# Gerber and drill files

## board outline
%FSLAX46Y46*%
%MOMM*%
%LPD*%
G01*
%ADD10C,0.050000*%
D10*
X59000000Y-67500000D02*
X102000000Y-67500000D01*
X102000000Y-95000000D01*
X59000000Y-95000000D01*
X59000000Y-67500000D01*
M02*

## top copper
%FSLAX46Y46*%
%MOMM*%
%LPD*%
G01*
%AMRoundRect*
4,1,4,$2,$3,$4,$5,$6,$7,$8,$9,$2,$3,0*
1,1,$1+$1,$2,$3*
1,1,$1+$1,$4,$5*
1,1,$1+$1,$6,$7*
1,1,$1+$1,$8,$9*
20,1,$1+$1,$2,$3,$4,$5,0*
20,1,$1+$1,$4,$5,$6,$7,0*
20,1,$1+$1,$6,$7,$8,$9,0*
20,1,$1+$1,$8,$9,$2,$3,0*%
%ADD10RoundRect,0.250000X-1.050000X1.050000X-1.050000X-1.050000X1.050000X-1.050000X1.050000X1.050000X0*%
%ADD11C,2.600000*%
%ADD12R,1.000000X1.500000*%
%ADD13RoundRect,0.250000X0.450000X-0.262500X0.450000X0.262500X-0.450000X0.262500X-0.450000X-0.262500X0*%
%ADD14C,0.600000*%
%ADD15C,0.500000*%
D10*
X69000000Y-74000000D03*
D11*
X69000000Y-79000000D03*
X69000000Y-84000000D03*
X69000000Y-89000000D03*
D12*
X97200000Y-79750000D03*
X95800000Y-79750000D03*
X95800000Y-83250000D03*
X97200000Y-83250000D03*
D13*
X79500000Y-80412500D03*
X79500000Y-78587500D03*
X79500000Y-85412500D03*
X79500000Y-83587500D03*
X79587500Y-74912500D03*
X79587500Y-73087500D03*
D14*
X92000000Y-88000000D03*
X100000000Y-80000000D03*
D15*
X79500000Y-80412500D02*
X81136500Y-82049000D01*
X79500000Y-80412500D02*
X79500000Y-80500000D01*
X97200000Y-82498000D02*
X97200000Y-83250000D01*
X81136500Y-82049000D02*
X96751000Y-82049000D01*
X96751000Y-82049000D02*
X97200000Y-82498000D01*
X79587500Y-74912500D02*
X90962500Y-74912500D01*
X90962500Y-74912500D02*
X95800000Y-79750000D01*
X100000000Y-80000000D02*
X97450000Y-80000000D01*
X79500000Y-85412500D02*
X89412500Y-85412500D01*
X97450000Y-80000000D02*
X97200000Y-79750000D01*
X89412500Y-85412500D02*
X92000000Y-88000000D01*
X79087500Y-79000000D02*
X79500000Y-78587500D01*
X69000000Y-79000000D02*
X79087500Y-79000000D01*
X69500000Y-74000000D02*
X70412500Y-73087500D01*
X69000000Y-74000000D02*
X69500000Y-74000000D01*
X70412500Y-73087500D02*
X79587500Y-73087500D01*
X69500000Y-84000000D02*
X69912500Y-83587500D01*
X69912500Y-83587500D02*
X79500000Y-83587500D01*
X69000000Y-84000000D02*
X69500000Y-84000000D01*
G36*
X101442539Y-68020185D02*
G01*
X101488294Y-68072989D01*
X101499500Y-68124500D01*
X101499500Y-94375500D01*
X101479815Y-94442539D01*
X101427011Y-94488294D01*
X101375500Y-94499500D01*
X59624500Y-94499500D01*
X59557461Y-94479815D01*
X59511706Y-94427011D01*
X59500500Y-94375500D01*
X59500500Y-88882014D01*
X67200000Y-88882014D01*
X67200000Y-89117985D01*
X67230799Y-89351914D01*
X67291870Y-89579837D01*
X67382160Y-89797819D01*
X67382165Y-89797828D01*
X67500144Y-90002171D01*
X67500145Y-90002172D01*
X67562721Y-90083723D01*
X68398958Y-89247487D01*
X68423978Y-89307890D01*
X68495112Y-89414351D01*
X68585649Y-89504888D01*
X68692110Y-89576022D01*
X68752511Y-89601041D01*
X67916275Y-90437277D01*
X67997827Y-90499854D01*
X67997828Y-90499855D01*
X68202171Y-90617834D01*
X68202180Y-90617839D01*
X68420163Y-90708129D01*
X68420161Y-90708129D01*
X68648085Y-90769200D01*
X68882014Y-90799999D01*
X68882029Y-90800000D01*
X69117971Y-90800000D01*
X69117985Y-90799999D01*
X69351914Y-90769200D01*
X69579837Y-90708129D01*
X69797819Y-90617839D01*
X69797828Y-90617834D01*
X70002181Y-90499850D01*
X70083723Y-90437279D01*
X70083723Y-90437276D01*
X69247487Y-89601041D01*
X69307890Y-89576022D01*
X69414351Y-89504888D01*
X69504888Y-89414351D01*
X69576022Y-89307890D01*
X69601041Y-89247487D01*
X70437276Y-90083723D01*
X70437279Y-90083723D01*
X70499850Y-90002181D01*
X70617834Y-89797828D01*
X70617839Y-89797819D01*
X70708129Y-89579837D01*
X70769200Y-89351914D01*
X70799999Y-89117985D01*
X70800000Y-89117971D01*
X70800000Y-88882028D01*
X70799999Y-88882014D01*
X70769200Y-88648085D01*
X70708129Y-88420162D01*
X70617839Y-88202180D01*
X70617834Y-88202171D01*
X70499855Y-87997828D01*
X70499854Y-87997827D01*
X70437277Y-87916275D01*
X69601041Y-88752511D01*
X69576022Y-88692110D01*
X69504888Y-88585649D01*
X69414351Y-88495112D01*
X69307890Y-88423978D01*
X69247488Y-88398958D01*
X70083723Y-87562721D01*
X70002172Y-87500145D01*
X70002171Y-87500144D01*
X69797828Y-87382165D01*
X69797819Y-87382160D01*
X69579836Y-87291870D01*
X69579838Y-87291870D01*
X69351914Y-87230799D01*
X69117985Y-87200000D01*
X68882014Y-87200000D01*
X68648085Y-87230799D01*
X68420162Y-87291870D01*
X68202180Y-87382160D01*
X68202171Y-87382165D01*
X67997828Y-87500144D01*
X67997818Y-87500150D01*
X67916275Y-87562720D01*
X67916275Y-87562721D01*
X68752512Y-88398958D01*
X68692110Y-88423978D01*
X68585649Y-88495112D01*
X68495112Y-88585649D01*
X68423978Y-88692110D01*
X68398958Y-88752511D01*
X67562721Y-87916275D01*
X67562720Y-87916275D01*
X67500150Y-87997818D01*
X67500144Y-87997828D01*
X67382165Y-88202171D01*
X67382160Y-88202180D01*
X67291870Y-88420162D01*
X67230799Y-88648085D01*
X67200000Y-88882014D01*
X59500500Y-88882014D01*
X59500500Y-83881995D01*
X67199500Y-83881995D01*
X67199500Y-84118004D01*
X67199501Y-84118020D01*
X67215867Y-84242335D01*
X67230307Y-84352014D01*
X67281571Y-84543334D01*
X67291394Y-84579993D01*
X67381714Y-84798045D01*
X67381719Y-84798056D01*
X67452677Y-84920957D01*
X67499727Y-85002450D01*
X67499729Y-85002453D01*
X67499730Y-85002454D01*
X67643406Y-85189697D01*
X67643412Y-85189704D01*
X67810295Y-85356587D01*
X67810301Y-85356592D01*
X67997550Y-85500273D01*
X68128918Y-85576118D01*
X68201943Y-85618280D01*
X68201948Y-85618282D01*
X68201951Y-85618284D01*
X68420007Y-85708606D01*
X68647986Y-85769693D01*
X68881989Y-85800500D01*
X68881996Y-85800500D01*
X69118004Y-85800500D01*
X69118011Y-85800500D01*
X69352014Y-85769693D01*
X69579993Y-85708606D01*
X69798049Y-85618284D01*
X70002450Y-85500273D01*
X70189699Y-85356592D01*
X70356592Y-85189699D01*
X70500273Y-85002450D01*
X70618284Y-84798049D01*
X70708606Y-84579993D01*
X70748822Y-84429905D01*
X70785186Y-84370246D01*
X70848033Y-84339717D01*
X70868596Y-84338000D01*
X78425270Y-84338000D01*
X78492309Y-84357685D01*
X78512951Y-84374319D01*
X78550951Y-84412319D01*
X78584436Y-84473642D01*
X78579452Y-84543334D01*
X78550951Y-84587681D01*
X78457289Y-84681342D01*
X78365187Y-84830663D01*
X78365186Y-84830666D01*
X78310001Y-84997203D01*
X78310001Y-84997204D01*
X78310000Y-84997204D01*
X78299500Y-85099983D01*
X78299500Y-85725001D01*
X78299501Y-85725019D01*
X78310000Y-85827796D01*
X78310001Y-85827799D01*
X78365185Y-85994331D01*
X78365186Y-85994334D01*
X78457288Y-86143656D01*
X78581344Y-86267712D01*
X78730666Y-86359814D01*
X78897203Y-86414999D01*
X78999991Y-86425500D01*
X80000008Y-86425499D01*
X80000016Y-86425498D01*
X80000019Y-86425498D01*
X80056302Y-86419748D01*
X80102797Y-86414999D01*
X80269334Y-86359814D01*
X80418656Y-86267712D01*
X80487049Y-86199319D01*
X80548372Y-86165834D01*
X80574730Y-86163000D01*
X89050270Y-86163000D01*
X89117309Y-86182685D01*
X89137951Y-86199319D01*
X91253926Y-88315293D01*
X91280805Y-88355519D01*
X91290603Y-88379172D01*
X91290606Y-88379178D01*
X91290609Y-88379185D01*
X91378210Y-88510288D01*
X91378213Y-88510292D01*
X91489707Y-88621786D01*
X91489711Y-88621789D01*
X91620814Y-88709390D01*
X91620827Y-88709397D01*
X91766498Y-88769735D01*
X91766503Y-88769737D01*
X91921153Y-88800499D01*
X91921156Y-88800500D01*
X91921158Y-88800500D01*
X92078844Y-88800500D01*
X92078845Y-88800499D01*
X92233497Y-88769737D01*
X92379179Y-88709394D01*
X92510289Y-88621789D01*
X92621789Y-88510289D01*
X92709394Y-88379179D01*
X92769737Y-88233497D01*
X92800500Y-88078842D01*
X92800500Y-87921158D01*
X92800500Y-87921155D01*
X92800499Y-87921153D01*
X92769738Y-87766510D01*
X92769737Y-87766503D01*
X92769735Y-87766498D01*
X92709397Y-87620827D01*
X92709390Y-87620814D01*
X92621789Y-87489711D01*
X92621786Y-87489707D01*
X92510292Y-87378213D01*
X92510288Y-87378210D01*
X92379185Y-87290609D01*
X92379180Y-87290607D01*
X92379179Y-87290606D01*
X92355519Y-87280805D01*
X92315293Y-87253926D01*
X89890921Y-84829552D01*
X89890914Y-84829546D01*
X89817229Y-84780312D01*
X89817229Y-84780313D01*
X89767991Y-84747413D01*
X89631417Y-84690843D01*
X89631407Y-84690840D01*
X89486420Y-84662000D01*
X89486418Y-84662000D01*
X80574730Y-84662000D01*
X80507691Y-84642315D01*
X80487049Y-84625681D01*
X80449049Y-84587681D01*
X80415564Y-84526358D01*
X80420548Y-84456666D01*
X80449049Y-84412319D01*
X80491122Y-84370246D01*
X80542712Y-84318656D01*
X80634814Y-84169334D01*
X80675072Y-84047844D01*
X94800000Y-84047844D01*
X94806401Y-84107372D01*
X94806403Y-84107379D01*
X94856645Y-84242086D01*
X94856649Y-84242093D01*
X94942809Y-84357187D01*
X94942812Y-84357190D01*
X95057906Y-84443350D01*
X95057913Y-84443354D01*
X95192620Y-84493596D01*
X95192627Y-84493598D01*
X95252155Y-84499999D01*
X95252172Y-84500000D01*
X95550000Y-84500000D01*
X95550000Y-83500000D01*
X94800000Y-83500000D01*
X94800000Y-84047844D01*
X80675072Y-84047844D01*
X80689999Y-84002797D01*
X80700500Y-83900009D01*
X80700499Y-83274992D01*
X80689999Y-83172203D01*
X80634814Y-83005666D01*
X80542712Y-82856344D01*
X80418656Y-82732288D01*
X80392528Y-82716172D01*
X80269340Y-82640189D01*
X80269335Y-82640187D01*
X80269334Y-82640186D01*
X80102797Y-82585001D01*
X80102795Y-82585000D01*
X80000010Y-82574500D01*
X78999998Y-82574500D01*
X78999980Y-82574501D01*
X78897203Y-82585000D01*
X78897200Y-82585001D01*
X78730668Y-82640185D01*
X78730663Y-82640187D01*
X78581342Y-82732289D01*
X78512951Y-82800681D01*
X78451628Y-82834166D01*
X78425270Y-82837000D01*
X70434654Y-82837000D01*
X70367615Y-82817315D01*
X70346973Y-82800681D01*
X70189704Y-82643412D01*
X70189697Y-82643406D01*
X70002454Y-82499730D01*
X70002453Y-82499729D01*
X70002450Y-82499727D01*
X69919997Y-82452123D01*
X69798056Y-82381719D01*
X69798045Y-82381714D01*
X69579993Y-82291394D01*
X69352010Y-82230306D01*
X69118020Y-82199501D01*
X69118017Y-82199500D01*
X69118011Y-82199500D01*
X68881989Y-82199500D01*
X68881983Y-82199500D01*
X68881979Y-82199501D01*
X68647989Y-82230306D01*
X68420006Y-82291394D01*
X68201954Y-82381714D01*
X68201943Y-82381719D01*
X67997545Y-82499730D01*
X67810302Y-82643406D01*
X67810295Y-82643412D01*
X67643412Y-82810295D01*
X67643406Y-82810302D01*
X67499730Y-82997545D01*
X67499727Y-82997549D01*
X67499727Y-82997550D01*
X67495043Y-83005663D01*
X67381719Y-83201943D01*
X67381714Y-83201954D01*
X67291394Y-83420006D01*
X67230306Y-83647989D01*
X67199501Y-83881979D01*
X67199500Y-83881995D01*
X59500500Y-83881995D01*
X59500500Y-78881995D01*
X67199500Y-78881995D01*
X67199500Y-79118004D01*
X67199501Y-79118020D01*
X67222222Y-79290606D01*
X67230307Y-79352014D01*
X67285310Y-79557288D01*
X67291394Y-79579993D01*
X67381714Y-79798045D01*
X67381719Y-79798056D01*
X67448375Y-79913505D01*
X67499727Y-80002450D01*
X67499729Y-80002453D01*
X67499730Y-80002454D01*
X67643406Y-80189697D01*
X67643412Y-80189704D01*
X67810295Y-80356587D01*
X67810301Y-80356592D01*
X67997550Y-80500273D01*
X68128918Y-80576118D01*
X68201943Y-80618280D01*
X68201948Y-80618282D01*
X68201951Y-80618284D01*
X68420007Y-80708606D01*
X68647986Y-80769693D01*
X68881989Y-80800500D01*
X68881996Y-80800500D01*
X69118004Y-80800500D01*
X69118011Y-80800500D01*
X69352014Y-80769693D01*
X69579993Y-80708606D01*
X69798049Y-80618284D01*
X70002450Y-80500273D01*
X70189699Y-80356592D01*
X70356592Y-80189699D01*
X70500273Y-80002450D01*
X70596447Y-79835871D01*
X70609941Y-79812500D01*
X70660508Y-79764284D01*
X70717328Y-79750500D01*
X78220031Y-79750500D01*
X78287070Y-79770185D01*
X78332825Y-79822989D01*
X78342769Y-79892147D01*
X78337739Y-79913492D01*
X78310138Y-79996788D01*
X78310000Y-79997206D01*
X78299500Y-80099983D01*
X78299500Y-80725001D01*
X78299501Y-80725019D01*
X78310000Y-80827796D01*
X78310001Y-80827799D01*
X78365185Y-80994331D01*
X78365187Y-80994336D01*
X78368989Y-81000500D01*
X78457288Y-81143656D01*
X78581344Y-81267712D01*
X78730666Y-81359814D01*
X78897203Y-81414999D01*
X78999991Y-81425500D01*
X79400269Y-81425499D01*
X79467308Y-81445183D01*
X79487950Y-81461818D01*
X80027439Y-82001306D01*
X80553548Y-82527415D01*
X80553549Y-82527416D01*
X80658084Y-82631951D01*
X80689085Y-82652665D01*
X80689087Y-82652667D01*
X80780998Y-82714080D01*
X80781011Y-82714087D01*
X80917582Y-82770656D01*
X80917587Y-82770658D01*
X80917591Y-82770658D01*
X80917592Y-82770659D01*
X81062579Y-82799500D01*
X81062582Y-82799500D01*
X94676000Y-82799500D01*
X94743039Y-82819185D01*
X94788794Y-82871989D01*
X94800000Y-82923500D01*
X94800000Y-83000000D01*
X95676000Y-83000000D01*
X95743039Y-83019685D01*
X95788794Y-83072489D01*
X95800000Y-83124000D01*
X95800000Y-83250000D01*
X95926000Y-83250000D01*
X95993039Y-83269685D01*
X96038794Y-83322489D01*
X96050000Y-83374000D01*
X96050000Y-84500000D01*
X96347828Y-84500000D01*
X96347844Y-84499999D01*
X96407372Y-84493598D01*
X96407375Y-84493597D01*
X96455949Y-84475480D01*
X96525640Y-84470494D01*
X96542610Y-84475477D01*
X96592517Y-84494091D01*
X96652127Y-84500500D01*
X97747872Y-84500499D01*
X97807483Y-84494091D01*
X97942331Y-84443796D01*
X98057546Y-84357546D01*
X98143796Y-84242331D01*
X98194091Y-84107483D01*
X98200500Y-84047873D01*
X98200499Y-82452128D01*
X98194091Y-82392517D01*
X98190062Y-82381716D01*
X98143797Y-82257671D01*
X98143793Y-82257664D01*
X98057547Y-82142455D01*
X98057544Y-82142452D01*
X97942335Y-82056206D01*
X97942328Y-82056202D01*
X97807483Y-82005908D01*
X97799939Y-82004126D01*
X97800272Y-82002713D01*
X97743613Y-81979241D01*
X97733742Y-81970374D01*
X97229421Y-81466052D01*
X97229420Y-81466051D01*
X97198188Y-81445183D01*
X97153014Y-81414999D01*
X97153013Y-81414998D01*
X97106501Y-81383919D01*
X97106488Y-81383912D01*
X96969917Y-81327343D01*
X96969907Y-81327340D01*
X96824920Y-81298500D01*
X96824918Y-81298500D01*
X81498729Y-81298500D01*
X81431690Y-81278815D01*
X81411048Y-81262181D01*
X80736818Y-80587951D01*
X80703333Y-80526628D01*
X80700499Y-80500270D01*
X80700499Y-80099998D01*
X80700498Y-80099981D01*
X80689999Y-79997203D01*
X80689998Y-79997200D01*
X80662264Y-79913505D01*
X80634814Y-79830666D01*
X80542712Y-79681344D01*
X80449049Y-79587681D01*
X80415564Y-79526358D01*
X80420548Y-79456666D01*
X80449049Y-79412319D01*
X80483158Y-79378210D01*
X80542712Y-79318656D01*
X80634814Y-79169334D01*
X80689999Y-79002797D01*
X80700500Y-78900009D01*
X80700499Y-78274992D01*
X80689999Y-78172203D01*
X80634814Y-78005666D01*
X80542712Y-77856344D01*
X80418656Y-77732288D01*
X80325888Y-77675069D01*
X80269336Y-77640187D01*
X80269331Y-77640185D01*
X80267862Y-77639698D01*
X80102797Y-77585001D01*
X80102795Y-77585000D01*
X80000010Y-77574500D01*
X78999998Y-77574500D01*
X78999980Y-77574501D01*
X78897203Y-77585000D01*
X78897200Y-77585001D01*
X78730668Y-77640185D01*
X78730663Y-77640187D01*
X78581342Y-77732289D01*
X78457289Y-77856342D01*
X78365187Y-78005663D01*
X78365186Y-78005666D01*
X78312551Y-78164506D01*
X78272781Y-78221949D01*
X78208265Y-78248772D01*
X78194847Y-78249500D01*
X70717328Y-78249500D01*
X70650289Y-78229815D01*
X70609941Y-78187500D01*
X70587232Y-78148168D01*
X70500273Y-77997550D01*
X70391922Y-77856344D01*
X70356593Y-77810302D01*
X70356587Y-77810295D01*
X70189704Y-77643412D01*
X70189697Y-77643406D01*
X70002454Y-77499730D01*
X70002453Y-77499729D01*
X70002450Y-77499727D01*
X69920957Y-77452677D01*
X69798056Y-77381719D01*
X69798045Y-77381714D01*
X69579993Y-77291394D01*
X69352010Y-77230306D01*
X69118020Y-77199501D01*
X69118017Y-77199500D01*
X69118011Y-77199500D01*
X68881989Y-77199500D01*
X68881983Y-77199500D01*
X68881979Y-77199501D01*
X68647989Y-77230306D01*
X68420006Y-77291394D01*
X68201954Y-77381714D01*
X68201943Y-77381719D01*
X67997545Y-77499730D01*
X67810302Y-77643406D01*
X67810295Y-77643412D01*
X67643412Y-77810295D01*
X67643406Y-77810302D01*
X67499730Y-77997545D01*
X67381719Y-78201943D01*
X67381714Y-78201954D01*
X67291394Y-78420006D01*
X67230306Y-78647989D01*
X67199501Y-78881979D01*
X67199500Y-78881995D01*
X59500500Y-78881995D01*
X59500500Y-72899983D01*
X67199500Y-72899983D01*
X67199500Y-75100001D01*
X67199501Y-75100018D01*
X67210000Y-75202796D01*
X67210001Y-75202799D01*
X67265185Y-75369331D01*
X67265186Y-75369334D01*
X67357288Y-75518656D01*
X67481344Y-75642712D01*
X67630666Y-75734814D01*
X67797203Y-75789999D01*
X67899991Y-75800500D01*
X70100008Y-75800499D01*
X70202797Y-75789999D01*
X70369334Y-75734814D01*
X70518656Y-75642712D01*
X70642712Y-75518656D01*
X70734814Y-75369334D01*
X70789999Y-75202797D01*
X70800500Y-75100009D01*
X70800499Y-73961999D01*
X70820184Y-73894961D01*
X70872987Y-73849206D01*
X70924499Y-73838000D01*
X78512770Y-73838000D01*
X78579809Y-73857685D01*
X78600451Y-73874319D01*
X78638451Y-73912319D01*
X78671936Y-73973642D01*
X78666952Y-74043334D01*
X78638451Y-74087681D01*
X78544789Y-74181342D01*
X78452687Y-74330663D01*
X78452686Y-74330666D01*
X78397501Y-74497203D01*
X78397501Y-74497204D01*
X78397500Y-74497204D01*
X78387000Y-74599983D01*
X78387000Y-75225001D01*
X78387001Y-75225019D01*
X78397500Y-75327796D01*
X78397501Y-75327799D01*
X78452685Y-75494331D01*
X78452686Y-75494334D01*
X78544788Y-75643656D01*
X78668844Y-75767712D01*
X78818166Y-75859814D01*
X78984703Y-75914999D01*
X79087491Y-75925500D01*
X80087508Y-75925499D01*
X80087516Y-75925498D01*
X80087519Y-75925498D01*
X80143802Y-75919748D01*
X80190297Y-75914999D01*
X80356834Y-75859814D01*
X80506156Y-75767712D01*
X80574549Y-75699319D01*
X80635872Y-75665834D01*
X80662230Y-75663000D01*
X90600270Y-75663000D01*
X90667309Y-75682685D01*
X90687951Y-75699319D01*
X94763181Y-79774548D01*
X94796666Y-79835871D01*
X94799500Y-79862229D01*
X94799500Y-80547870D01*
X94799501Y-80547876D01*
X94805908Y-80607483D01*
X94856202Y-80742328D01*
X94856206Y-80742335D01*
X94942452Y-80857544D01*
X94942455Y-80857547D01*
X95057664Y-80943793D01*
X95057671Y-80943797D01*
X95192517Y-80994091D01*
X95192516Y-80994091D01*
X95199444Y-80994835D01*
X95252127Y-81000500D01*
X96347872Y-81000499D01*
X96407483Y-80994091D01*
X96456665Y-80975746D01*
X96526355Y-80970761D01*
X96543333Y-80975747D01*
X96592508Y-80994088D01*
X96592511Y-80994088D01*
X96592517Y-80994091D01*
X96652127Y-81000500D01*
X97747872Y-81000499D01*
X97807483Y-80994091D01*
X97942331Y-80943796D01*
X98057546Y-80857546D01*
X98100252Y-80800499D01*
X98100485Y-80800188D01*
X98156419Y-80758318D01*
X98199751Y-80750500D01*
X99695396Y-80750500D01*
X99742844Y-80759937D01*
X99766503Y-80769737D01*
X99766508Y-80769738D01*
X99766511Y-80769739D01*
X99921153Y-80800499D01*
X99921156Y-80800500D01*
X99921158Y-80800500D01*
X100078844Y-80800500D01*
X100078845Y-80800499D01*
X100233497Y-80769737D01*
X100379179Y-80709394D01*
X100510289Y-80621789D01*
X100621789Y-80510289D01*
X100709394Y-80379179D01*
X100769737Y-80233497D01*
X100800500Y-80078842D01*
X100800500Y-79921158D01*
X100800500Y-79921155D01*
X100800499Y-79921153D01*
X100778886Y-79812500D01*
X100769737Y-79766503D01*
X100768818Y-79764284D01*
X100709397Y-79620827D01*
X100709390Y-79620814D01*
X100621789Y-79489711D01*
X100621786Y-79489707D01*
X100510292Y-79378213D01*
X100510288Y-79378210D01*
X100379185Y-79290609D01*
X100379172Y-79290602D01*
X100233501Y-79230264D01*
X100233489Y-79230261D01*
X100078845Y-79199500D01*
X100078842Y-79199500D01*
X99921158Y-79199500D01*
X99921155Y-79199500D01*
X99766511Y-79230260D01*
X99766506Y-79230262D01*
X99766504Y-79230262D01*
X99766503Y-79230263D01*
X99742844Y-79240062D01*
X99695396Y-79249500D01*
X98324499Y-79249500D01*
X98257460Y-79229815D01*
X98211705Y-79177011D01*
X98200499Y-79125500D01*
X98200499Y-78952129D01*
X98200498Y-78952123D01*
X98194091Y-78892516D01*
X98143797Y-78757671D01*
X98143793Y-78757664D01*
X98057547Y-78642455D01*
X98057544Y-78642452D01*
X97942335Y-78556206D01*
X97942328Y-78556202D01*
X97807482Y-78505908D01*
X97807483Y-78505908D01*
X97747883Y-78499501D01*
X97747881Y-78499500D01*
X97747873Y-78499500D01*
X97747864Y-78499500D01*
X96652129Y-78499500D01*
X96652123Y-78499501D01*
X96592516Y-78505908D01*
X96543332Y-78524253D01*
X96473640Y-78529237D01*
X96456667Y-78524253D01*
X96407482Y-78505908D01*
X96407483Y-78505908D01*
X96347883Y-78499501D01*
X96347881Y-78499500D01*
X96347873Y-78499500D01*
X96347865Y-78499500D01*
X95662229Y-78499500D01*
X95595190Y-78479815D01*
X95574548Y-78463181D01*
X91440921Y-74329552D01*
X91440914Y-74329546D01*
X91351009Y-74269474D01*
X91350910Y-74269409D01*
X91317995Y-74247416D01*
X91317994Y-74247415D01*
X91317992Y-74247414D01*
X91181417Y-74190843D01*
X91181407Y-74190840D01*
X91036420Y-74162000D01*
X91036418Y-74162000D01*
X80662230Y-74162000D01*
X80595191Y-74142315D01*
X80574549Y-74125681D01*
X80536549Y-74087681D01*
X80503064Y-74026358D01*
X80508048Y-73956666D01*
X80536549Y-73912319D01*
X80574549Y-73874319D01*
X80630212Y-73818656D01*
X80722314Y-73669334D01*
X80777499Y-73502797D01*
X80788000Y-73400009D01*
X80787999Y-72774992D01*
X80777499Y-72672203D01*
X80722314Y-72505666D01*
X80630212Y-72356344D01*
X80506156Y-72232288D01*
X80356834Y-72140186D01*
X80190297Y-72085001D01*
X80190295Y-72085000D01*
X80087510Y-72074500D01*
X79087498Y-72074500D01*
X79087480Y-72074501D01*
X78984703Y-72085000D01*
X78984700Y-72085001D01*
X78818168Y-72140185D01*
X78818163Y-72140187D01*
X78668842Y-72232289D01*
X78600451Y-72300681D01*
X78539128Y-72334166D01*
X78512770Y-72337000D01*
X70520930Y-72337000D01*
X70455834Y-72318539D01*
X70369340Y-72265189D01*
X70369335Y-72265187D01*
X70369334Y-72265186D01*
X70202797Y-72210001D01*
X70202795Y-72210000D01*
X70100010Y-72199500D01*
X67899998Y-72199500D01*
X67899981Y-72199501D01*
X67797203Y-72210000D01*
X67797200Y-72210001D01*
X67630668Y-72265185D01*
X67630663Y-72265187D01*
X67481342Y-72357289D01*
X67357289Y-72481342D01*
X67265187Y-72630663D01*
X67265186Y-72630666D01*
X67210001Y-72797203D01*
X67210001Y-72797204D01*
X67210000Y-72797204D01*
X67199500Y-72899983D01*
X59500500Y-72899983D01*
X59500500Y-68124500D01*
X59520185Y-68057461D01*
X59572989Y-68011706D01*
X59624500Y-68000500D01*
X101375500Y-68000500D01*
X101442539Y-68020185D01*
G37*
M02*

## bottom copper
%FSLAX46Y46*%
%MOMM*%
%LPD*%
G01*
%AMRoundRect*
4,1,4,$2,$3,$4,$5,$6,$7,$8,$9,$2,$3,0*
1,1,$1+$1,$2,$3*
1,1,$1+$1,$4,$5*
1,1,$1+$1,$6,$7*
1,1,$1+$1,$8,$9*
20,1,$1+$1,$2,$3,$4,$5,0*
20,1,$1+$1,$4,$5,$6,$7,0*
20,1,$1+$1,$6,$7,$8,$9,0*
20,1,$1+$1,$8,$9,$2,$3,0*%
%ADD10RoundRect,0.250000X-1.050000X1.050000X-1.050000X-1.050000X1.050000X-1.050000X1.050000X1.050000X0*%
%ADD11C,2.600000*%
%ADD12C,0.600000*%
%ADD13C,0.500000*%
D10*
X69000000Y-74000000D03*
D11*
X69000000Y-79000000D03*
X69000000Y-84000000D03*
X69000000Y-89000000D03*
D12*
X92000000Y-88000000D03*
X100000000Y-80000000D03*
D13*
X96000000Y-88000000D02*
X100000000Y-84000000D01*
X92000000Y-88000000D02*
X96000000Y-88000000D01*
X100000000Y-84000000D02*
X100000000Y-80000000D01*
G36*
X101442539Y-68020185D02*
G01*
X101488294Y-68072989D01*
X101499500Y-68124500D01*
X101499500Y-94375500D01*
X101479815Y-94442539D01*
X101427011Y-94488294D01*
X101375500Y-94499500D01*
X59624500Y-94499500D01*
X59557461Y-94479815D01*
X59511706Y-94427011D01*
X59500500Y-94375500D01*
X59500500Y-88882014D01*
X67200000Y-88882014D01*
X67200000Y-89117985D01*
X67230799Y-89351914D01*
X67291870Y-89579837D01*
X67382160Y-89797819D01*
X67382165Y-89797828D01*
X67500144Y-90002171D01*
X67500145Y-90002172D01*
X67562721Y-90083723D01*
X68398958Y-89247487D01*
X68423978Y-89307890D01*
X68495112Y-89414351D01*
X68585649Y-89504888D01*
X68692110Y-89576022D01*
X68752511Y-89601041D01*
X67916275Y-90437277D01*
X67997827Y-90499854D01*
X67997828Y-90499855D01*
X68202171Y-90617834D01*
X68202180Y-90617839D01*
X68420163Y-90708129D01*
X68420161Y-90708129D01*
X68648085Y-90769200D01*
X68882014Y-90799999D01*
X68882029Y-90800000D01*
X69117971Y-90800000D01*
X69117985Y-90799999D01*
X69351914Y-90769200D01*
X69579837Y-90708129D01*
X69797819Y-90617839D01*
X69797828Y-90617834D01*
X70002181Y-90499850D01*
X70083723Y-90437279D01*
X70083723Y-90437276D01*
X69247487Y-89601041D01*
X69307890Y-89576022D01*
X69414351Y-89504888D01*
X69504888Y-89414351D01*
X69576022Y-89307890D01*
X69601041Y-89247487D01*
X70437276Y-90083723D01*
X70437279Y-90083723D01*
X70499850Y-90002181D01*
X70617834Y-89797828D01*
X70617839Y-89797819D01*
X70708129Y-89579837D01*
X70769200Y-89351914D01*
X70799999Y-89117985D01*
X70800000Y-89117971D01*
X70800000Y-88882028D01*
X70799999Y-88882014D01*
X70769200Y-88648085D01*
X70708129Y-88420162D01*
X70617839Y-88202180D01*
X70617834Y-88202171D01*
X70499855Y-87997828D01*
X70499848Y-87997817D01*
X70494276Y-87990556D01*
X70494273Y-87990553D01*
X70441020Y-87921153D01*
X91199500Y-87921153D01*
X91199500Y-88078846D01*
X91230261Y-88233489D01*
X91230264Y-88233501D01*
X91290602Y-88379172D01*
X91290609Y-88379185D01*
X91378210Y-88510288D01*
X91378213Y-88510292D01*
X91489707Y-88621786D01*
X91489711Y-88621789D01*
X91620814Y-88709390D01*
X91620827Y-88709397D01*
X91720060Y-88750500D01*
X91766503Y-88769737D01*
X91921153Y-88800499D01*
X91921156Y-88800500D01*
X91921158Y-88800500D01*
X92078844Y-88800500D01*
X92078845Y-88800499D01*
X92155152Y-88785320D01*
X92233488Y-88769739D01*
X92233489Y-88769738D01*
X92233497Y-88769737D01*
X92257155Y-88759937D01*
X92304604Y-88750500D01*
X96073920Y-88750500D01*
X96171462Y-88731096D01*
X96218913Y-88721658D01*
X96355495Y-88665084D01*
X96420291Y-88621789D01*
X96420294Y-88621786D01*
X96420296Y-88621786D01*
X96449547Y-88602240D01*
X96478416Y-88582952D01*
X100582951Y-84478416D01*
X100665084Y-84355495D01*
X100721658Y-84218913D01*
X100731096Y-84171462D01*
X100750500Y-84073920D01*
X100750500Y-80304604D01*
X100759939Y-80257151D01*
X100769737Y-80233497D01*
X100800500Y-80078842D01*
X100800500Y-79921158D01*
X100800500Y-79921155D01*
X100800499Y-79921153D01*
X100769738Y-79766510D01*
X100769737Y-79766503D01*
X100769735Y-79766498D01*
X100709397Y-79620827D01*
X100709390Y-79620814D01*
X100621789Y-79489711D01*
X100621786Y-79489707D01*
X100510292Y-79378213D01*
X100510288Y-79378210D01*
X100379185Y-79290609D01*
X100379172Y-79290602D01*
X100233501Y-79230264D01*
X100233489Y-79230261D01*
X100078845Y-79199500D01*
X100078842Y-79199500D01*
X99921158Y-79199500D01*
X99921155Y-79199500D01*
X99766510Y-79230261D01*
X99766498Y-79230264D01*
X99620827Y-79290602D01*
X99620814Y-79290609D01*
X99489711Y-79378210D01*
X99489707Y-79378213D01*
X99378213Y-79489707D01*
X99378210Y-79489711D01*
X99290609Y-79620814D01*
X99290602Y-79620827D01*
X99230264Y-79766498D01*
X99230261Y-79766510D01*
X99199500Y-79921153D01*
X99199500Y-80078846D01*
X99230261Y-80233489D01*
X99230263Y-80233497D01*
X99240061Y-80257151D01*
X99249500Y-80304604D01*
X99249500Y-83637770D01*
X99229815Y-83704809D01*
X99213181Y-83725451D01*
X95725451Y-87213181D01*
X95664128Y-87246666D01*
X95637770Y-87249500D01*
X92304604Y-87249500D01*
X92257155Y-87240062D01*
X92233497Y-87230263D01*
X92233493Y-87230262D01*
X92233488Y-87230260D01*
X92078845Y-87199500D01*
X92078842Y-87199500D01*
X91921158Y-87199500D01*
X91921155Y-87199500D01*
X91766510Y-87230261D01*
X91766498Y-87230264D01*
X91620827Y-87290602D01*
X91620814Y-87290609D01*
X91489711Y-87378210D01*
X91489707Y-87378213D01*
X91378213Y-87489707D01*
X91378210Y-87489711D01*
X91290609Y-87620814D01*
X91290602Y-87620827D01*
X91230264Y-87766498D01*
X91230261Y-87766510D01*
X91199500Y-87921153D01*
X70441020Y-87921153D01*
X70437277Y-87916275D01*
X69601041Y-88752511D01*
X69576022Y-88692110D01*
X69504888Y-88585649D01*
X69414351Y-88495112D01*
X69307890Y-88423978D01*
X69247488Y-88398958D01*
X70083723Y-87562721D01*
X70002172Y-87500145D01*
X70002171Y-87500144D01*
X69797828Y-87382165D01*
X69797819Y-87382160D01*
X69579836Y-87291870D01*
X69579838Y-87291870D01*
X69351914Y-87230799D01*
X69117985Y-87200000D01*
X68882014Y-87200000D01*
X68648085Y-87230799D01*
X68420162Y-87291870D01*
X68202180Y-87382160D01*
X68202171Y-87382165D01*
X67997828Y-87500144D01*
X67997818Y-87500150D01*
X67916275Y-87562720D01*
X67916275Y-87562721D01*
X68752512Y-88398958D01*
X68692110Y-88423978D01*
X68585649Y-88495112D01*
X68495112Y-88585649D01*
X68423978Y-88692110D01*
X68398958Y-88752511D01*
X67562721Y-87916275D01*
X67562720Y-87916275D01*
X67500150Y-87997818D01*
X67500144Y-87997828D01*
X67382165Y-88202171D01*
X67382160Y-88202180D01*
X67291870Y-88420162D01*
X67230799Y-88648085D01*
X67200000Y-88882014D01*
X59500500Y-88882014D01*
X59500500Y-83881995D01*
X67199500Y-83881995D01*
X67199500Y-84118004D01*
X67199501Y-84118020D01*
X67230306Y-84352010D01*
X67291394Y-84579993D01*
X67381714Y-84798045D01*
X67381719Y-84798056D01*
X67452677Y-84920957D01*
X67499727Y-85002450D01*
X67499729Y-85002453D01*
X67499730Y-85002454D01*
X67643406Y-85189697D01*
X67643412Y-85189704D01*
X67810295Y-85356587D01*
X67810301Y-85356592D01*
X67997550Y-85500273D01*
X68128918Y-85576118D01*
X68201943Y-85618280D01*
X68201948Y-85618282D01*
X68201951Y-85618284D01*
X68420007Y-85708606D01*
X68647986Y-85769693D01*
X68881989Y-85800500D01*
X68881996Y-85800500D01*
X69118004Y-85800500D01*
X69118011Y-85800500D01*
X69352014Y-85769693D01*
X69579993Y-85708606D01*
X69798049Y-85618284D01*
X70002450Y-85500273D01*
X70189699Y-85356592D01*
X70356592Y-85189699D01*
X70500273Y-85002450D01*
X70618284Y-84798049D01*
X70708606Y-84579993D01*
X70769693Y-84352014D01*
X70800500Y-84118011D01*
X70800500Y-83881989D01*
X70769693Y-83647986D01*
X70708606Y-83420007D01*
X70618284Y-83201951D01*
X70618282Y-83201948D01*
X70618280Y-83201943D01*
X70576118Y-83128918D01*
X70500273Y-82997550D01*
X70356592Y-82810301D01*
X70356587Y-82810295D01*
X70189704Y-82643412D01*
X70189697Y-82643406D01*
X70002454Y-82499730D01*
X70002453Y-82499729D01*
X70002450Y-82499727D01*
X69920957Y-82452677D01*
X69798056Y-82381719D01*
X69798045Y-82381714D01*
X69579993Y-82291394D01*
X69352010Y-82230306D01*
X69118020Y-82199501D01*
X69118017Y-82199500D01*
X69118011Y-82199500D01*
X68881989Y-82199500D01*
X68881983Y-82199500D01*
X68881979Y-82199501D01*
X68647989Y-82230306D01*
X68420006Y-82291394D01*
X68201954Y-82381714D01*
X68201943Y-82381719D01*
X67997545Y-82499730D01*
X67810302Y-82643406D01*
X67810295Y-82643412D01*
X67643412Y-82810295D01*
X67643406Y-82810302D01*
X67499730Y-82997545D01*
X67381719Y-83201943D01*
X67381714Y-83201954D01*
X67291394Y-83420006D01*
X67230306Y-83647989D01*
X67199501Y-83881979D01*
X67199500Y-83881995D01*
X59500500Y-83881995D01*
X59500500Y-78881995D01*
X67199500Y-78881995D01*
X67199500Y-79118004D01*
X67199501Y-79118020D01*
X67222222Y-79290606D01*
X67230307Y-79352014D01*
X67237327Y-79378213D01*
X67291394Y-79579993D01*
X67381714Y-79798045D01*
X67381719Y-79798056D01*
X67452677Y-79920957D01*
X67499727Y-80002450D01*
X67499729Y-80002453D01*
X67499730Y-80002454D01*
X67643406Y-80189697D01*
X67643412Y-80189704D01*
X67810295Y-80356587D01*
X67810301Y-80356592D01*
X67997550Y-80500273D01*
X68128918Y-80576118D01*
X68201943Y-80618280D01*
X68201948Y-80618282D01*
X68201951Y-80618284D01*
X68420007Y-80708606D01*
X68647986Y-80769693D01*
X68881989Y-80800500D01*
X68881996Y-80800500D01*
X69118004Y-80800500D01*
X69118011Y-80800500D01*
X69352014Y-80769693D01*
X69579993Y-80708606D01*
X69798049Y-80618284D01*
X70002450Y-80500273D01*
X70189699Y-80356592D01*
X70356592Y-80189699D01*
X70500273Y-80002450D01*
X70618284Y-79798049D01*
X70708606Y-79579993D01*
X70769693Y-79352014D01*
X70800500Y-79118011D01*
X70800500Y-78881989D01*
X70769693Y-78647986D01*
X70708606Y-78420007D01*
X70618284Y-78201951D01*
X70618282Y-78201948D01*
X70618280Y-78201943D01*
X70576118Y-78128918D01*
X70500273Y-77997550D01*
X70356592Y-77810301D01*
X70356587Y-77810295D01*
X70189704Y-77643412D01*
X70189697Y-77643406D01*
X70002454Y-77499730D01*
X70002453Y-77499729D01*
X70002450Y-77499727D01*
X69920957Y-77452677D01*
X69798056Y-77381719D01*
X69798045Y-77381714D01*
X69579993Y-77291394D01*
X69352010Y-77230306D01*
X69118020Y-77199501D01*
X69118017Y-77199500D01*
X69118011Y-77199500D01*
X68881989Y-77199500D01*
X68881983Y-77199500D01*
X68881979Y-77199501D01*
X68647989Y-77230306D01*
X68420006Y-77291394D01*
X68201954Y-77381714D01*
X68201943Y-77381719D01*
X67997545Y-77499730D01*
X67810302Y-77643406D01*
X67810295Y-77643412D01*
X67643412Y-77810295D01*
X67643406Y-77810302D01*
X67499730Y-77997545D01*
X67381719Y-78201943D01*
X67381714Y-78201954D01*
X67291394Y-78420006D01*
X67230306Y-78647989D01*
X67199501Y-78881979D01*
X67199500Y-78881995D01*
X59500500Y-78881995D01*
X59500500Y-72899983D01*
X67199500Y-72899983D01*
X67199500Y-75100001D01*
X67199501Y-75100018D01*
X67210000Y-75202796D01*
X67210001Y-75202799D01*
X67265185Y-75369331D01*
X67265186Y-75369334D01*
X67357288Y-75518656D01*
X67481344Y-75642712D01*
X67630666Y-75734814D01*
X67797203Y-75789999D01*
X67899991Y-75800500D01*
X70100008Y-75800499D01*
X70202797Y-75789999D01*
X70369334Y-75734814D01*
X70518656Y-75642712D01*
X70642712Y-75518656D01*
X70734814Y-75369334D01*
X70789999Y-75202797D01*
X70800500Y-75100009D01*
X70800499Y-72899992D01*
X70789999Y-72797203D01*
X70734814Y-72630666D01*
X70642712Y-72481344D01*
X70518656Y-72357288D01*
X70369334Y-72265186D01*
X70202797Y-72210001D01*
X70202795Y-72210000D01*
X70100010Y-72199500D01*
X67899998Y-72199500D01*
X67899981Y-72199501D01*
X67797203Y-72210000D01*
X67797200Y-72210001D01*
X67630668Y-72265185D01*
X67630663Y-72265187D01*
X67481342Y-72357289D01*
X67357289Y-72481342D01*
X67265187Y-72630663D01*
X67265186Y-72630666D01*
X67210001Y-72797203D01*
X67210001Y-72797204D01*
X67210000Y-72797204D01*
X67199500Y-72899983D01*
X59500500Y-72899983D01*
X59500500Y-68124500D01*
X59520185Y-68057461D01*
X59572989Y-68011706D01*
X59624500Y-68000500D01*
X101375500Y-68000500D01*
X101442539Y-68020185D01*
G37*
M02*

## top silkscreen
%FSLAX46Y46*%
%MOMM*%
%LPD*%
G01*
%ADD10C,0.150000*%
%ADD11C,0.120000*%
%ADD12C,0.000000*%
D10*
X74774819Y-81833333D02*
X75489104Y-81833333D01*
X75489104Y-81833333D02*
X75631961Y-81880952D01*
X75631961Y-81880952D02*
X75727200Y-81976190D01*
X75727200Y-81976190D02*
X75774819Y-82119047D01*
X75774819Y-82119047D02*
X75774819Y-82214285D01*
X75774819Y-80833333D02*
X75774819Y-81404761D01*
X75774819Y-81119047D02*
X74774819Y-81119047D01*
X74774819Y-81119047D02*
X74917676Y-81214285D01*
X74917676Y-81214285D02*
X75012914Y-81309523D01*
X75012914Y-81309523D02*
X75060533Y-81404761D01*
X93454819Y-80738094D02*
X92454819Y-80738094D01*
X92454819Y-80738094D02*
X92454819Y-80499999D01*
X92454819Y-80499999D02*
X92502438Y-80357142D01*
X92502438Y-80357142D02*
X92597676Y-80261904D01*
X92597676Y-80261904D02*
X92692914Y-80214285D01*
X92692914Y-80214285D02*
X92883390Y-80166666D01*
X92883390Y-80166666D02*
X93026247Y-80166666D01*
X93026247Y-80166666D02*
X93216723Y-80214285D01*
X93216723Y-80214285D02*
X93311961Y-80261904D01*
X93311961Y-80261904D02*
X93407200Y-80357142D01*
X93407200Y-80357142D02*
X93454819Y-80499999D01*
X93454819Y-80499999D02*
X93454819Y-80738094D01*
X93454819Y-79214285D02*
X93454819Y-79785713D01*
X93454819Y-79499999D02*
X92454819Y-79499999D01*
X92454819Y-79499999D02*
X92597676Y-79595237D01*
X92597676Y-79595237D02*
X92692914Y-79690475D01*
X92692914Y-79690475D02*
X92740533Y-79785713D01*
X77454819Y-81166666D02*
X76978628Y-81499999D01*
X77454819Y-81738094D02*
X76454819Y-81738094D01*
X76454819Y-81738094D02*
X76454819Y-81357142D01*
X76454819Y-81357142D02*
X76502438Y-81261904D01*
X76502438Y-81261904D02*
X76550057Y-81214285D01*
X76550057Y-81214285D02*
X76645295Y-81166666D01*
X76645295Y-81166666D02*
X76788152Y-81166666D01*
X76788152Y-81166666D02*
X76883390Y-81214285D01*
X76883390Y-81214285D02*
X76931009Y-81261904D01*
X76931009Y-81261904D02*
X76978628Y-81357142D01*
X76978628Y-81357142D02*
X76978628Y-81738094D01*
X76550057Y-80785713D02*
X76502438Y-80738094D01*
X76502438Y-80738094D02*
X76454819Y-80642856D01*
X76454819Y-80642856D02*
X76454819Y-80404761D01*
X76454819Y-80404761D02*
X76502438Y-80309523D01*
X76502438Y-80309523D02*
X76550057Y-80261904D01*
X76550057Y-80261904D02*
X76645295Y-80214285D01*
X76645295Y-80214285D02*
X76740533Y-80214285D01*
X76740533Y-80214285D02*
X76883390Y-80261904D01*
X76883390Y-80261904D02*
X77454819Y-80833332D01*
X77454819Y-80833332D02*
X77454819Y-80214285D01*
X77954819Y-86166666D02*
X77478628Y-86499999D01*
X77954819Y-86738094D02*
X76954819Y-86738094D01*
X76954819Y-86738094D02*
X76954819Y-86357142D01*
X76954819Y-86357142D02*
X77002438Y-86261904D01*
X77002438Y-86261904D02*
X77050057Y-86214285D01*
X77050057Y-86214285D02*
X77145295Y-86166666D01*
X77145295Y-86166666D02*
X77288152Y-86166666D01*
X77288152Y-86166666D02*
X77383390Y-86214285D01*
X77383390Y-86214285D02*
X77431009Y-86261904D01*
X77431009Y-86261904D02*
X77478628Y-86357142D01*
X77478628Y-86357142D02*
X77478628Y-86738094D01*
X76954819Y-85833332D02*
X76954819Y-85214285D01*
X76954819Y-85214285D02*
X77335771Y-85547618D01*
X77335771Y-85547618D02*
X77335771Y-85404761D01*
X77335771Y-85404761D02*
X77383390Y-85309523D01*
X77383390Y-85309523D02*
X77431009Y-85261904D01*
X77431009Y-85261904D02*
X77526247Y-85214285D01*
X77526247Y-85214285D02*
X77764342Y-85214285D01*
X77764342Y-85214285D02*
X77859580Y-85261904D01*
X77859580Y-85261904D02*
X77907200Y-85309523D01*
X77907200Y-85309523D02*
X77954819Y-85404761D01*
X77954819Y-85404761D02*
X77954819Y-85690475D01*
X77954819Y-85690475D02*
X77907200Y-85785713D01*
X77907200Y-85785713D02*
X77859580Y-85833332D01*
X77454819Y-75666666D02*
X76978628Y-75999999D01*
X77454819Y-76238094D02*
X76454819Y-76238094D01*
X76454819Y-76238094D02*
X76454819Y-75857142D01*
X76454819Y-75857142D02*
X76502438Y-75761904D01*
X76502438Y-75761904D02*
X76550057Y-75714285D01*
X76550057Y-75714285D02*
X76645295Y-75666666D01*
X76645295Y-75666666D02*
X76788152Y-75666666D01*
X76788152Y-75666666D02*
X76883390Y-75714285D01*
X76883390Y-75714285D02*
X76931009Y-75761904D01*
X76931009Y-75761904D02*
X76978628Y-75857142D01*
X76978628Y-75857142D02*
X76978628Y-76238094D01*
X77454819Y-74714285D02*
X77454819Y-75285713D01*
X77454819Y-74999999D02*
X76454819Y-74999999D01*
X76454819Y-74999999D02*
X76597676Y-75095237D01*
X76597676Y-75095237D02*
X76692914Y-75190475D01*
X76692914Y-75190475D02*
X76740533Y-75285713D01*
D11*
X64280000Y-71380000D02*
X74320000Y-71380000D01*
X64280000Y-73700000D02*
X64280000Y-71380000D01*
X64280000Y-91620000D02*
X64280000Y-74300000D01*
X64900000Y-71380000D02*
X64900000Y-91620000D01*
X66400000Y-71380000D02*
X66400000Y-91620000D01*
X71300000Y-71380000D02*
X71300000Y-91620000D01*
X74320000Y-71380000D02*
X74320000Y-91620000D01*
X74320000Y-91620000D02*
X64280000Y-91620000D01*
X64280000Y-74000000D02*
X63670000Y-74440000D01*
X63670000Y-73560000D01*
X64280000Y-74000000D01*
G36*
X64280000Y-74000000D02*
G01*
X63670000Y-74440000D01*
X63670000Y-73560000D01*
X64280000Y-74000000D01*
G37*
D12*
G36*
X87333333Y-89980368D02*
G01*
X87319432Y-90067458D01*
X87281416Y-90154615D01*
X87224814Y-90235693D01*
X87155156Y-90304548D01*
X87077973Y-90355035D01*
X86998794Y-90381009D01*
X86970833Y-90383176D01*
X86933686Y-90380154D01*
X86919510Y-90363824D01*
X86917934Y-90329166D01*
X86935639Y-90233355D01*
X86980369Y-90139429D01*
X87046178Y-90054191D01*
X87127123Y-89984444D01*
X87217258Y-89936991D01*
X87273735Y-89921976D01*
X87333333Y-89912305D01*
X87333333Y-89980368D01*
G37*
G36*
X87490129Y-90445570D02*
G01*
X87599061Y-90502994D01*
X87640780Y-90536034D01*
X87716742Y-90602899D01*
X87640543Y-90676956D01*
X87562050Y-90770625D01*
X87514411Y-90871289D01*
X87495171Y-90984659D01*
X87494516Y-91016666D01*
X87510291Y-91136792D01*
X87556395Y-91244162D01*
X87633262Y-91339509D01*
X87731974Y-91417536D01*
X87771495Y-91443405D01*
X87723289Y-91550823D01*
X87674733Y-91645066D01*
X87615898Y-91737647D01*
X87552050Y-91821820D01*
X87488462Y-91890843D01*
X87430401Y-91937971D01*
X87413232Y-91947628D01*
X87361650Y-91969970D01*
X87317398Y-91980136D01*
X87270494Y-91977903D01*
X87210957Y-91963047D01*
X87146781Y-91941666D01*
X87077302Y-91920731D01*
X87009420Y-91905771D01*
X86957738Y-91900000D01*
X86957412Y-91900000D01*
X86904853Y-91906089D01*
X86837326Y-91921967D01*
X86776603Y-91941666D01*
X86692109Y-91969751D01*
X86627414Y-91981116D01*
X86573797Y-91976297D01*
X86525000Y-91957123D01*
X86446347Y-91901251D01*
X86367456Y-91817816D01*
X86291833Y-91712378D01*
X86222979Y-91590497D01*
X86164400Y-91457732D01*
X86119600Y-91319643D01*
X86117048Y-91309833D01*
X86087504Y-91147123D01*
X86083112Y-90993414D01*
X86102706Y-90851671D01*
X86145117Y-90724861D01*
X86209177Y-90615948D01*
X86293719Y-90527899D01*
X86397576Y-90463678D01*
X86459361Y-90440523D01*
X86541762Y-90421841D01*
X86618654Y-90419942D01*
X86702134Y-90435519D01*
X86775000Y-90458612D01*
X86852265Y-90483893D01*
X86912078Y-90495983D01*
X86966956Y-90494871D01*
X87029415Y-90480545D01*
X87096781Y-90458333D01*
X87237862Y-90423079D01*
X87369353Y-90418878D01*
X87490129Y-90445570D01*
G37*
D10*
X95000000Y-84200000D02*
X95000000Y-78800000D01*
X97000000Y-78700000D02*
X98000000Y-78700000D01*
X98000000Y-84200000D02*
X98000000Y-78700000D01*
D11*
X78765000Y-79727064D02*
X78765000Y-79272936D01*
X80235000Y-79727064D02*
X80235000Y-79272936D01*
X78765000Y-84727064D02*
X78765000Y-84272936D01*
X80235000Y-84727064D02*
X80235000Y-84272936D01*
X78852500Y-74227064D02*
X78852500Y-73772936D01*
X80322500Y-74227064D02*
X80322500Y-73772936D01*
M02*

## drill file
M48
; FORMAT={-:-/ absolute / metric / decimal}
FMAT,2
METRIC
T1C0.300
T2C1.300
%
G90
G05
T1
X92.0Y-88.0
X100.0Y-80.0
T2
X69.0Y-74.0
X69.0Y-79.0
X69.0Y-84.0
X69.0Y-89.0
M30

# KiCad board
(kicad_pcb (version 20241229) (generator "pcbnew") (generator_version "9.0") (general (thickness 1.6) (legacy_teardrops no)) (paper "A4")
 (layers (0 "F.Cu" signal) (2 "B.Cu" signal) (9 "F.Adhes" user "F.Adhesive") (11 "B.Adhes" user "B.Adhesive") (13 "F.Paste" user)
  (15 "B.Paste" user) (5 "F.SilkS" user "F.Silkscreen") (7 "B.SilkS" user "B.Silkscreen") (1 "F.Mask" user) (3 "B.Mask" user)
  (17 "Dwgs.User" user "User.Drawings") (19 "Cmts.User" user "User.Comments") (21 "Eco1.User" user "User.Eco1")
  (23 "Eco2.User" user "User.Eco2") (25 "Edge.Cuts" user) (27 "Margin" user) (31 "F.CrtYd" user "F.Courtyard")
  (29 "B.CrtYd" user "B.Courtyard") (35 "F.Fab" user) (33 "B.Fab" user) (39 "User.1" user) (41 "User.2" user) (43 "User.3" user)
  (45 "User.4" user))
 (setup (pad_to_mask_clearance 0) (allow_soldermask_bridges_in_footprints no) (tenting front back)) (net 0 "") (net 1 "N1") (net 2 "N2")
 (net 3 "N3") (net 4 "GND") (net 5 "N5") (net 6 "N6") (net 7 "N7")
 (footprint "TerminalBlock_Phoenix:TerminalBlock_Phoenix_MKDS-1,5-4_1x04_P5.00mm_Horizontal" (layer "F.Cu") (at 69 74 -90)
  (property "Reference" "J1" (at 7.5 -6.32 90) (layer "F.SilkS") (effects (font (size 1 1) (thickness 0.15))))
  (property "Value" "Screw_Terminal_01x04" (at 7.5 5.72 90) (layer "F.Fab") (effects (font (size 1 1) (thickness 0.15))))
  (fp_line (start -2.62 4.72) (end -2.62 -5.32) (stroke (width 0.12) (type solid)) (layer "F.SilkS"))
  (fp_line (start -0.3 4.72) (end -2.62 4.72) (stroke (width 0.12) (type solid)) (layer "F.SilkS"))
  (fp_line (start 17.62 4.72) (end 0.3 4.72) (stroke (width 0.12) (type solid)) (layer "F.SilkS"))
  (fp_line (start -2.62 4.1) (end 17.62 4.1) (stroke (width 0.12) (type solid)) (layer "F.SilkS"))
  (fp_line (start -2.62 2.6) (end 17.62 2.6) (stroke (width 0.12) (type solid)) (layer "F.SilkS"))
  (fp_line (start -2.62 -2.3) (end 17.62 -2.3) (stroke (width 0.12) (type solid)) (layer "F.SilkS"))
  (fp_line (start -2.62 -5.32) (end 17.62 -5.32) (stroke (width 0.12) (type solid)) (layer "F.SilkS"))
  (fp_line (start 17.62 -5.32) (end 17.62 4.72) (stroke (width 0.12) (type solid)) (layer "F.SilkS"))
  (fp_poly (pts (xy 0 4.72) (xy 0.44 5.33) (xy -0.44 5.33)) (stroke (width 0.12) (type solid)) (fill yes) (layer "F.SilkS"))
  (pad "1" thru_hole roundrect (at 0 0 270) (size 2.6 2.6) (drill 1.3) (layers "*.Cu" "*.Mask") (remove_unused_layers no)
   (roundrect_rratio 0.096154) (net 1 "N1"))
  (pad "2" thru_hole circle (at 5 0 270) (size 2.6 2.6) (drill 1.3) (layers "*.Cu" "*.Mask") (remove_unused_layers no) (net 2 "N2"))
  (pad "3" thru_hole circle (at 10 0 270) (size 2.6 2.6) (drill 1.3) (layers "*.Cu" "*.Mask") (remove_unused_layers no) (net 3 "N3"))
  (pad "4" thru_hole circle (at 15 0 270) (size 2.6 2.6) (drill 1.3) (layers "*.Cu" "*.Mask") (remove_unused_layers no) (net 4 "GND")))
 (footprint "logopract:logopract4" (layer "F.Cu") (at 87 91)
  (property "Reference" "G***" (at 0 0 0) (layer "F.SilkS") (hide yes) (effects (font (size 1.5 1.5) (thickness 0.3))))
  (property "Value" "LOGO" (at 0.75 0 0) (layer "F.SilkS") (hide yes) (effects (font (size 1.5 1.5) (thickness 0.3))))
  (fp_poly
   (pts (xy 0.333333 -1.019632) (xy 0.319432 -0.932542) (xy 0.281416 -0.845385) (xy 0.224814 -0.764307) (xy 0.155156 -0.695452)
    (xy 0.077973 -0.644965) (xy -0.001206 -0.618991) (xy -0.029167 -0.616824) (xy -0.066314 -0.619846) (xy -0.08049 -0.636176)
    (xy -0.082066 -0.670834) (xy -0.064361 -0.766645) (xy -0.019631 -0.860571) (xy 0.046178 -0.945809) (xy 0.127123 -1.015556)
    (xy 0.217258 -1.063009) (xy 0.273735 -1.078024) (xy 0.333333 -1.087695))
   (stroke (width 0) (type solid)) (fill yes) (layer "F.SilkS"))
  (fp_poly
   (pts (xy 0.490129 -0.55443) (xy 0.599061 -0.497006) (xy 0.64078 -0.463966) (xy 0.716742 -0.397101) (xy 0.640543 -0.323044)
    (xy 0.56205 -0.229375) (xy 0.514411 -0.128711) (xy 0.495171 -0.015341) (xy 0.494516 0.016666) (xy 0.510291 0.136792)
    (xy 0.556395 0.244162) (xy 0.633262 0.339509) (xy 0.731974 0.417536) (xy 0.771495 0.443405) (xy 0.723289 0.550823)
    (xy 0.674733 0.645066) (xy 0.615898 0.737647) (xy 0.55205 0.82182) (xy 0.488462 0.890843) (xy 0.430401 0.937971) (xy 0.413232 0.947628)
    (xy 0.36165 0.96997) (xy 0.317398 0.980136) (xy 0.270494 0.977903) (xy 0.210957 0.963047) (xy 0.146781 0.941666) (xy 0.077302 0.920731)
    (xy 0.00942 0.905771) (xy -0.042262 0.9) (xy -0.042588 0.9) (xy -0.095147 0.906089) (xy -0.162674 0.921967) (xy -0.223397 0.941666)
    (xy -0.307891 0.969751) (xy -0.372586 0.981116) (xy -0.426203 0.976297) (xy -0.475 0.957123) (xy -0.553653 0.901251)
    (xy -0.632544 0.817816) (xy -0.708167 0.712378) (xy -0.777021 0.590497) (xy -0.8356 0.457732) (xy -0.8804 0.319643)
    (xy -0.882952 0.309833) (xy -0.912496 0.147123) (xy -0.916888 -0.006586) (xy -0.897294 -0.148329) (xy -0.854883 -0.275139)
    (xy -0.790823 -0.384052) (xy -0.706281 -0.472101) (xy -0.602424 -0.536322) (xy -0.540639 -0.559477) (xy -0.458238 -0.578159)
    (xy -0.381346 -0.580058) (xy -0.297866 -0.564481) (xy -0.225 -0.541388) (xy -0.147735 -0.516107) (xy -0.087922 -0.504017)
    (xy -0.033044 -0.505129) (xy 0.029415 -0.519455) (xy 0.096781 -0.541667) (xy 0.237862 -0.576921) (xy 0.369353 -0.581122))
   (stroke (width 0) (type solid)) (fill yes) (layer "F.SilkS")))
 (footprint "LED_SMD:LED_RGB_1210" (layer "F.Cu") (at 96.5 81.5 -90)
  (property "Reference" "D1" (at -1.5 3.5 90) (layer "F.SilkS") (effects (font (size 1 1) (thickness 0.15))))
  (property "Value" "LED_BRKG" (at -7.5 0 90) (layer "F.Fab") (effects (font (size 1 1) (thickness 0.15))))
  (fp_line (start 2.7 1.5) (end -2.7 1.5) (stroke (width 0.15) (type solid)) (layer "F.SilkS"))
  (fp_line (start -2.8 -0.5) (end -2.8 -1.5) (stroke (width 0.15) (type solid)) (layer "F.SilkS"))
  (fp_line (start 2.7 -1.5) (end -2.8 -1.5) (stroke (width 0.15) (type solid)) (layer "F.SilkS"))
  (pad "1" smd rect (at -1.75 -0.7 90) (size 1.5 1) (layers "F.Cu" "F.Mask" "F.Paste") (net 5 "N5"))
  (pad "2" smd rect (at -1.75 0.7 90) (size 1.5 1) (layers "F.Cu" "F.Mask" "F.Paste") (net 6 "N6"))
  (pad "3" smd rect (at 1.75 0.7 90) (size 1.5 1) (layers "F.Cu" "F.Mask" "F.Paste") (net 4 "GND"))
  (pad "4" smd rect (at 1.75 -0.7 90) (size 1.5 1) (layers "F.Cu" "F.Mask" "F.Paste") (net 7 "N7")))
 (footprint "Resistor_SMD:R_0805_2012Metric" (layer "F.Cu") (at 79.5 79.5 90)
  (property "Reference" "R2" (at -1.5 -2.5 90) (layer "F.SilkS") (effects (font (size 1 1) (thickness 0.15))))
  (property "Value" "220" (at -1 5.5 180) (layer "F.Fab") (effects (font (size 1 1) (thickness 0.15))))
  (fp_line (start -0.227064 -0.735) (end 0.227064 -0.735) (stroke (width 0.12) (type solid)) (layer "F.SilkS"))
  (fp_line (start -0.227064 0.735) (end 0.227064 0.735) (stroke (width 0.12) (type solid)) (layer "F.SilkS"))
  (pad "1" smd roundrect (at -0.9125 0 90) (size 1.025 1.4) (layers "F.Cu" "F.Mask" "F.Paste") (roundrect_rratio 0.243902) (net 7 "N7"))
  (pad "2" smd roundrect (at 0.9125 0 90) (size 1.025 1.4) (layers "F.Cu" "F.Mask" "F.Paste") (roundrect_rratio 0.243902) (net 2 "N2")))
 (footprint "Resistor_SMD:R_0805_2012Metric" (layer "F.Cu") (at 79.5 84.5 90)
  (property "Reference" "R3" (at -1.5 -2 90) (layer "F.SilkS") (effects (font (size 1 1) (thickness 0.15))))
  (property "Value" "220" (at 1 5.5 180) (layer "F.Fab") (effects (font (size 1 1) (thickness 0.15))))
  (fp_line (start -0.227064 -0.735) (end 0.227064 -0.735) (stroke (width 0.12) (type solid)) (layer "F.SilkS"))
  (fp_line (start -0.227064 0.735) (end 0.227064 0.735) (stroke (width 0.12) (type solid)) (layer "F.SilkS"))
  (pad "1" smd roundrect (at -0.9125 0 90) (size 1.025 1.4) (layers "F.Cu" "F.Mask" "F.Paste") (roundrect_rratio 0.243902) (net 5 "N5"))
  (pad "2" smd roundrect (at 0.9125 0 90) (size 1.025 1.4) (layers "F.Cu" "F.Mask" "F.Paste") (roundrect_rratio 0.243902) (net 3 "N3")))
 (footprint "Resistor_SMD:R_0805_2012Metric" (layer "F.Cu") (at 79.5875 74 90)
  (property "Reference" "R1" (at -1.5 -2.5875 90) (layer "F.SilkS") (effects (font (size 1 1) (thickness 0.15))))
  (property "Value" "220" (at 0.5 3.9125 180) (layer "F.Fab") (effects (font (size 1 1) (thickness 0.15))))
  (fp_line (start -0.227064 -0.735) (end 0.227064 -0.735) (stroke (width 0.12) (type solid)) (layer "F.SilkS"))
  (fp_line (start -0.227064 0.735) (end 0.227064 0.735) (stroke (width 0.12) (type solid)) (layer "F.SilkS"))
  (pad "1" smd roundrect (at -0.9125 0 90) (size 1.025 1.4) (layers "F.Cu" "F.Mask" "F.Paste") (roundrect_rratio 0.243902) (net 6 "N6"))
  (pad "2" smd roundrect (at 0.9125 0 90) (size 1.025 1.4) (layers "F.Cu" "F.Mask" "F.Paste") (roundrect_rratio 0.243902) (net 1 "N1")))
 (gr_rect (start 59 67.5) (end 102 95) (stroke (width 0.05) (type default)) (fill no) (layer "Edge.Cuts"))
 (segment (start 79.5 80.4125) (end 81.1365 82.049) (width 0.5) (layer "F.Cu") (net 7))
 (segment (start 79.5 80.4125) (end 79.5 80.5) (width 0.5) (layer "F.Cu") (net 7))
 (segment (start 97.2 82.498) (end 97.2 83.25) (width 0.5) (layer "F.Cu") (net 7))
 (segment (start 81.1365 82.049) (end 96.751 82.049) (width 0.5) (layer "F.Cu") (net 7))
 (segment (start 96.751 82.049) (end 97.2 82.498) (width 0.5) (layer "F.Cu") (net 7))
 (segment (start 79.5875 74.9125) (end 90.9625 74.9125) (width 0.5) (layer "F.Cu") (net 6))
 (segment (start 90.9625 74.9125) (end 95.8 79.75) (width 0.5) (layer "F.Cu") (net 6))
 (segment (start 100 80) (end 97.45 80) (width 0.5) (layer "F.Cu") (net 5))
 (segment (start 79.5 85.4125) (end 89.4125 85.4125) (width 0.5) (layer "F.Cu") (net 5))
 (segment (start 97.45 80) (end 97.2 79.75) (width 0.5) (layer "F.Cu") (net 5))
 (segment (start 89.4125 85.4125) (end 92 88) (width 0.5) (layer "F.Cu") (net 5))
 (via (at 92 88) (size 0.6) (drill 0.3) (layers "F.Cu" "B.Cu") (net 5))
 (via (at 100 80) (size 0.6) (drill 0.3) (layers "F.Cu" "B.Cu") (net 5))
 (segment (start 96 88) (end 100 84) (width 0.5) (layer "B.Cu") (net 5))
 (segment (start 92 88) (end 96 88) (width 0.5) (layer "B.Cu") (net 5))
 (segment (start 100 84) (end 100 80) (width 0.5) (layer "B.Cu") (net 5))
 (segment (start 79.0875 79) (end 79.5 78.5875) (width 0.5) (layer "F.Cu") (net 2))
 (segment (start 69 79) (end 79.0875 79) (width 0.5) (layer "F.Cu") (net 2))
 (segment (start 69.5 74) (end 70.4125 73.0875) (width 0.5) (layer "F.Cu") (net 1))
 (segment (start 69 74) (end 69.5 74) (width 0.5) (layer "F.Cu") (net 1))
 (segment (start 70.4125 73.0875) (end 79.5875 73.0875) (width 0.5) (layer "F.Cu") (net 1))
 (segment (start 69.5 84) (end 69.9125 83.5875) (width 0.5) (layer "F.Cu") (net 3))
 (segment (start 69.9125 83.5875) (end 79.5 83.5875) (width 0.5) (layer "F.Cu") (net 3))
 (segment (start 69 84) (end 69.5 84) (width 0.5) (layer "F.Cu") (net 3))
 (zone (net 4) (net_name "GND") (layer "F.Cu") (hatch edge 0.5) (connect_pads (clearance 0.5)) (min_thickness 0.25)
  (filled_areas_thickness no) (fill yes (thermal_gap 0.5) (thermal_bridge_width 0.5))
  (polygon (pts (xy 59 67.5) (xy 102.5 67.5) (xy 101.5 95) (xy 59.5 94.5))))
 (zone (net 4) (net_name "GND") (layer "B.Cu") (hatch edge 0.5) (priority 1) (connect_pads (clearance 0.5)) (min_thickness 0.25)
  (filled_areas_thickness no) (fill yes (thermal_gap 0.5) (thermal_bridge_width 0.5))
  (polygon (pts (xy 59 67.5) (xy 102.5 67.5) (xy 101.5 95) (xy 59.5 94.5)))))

